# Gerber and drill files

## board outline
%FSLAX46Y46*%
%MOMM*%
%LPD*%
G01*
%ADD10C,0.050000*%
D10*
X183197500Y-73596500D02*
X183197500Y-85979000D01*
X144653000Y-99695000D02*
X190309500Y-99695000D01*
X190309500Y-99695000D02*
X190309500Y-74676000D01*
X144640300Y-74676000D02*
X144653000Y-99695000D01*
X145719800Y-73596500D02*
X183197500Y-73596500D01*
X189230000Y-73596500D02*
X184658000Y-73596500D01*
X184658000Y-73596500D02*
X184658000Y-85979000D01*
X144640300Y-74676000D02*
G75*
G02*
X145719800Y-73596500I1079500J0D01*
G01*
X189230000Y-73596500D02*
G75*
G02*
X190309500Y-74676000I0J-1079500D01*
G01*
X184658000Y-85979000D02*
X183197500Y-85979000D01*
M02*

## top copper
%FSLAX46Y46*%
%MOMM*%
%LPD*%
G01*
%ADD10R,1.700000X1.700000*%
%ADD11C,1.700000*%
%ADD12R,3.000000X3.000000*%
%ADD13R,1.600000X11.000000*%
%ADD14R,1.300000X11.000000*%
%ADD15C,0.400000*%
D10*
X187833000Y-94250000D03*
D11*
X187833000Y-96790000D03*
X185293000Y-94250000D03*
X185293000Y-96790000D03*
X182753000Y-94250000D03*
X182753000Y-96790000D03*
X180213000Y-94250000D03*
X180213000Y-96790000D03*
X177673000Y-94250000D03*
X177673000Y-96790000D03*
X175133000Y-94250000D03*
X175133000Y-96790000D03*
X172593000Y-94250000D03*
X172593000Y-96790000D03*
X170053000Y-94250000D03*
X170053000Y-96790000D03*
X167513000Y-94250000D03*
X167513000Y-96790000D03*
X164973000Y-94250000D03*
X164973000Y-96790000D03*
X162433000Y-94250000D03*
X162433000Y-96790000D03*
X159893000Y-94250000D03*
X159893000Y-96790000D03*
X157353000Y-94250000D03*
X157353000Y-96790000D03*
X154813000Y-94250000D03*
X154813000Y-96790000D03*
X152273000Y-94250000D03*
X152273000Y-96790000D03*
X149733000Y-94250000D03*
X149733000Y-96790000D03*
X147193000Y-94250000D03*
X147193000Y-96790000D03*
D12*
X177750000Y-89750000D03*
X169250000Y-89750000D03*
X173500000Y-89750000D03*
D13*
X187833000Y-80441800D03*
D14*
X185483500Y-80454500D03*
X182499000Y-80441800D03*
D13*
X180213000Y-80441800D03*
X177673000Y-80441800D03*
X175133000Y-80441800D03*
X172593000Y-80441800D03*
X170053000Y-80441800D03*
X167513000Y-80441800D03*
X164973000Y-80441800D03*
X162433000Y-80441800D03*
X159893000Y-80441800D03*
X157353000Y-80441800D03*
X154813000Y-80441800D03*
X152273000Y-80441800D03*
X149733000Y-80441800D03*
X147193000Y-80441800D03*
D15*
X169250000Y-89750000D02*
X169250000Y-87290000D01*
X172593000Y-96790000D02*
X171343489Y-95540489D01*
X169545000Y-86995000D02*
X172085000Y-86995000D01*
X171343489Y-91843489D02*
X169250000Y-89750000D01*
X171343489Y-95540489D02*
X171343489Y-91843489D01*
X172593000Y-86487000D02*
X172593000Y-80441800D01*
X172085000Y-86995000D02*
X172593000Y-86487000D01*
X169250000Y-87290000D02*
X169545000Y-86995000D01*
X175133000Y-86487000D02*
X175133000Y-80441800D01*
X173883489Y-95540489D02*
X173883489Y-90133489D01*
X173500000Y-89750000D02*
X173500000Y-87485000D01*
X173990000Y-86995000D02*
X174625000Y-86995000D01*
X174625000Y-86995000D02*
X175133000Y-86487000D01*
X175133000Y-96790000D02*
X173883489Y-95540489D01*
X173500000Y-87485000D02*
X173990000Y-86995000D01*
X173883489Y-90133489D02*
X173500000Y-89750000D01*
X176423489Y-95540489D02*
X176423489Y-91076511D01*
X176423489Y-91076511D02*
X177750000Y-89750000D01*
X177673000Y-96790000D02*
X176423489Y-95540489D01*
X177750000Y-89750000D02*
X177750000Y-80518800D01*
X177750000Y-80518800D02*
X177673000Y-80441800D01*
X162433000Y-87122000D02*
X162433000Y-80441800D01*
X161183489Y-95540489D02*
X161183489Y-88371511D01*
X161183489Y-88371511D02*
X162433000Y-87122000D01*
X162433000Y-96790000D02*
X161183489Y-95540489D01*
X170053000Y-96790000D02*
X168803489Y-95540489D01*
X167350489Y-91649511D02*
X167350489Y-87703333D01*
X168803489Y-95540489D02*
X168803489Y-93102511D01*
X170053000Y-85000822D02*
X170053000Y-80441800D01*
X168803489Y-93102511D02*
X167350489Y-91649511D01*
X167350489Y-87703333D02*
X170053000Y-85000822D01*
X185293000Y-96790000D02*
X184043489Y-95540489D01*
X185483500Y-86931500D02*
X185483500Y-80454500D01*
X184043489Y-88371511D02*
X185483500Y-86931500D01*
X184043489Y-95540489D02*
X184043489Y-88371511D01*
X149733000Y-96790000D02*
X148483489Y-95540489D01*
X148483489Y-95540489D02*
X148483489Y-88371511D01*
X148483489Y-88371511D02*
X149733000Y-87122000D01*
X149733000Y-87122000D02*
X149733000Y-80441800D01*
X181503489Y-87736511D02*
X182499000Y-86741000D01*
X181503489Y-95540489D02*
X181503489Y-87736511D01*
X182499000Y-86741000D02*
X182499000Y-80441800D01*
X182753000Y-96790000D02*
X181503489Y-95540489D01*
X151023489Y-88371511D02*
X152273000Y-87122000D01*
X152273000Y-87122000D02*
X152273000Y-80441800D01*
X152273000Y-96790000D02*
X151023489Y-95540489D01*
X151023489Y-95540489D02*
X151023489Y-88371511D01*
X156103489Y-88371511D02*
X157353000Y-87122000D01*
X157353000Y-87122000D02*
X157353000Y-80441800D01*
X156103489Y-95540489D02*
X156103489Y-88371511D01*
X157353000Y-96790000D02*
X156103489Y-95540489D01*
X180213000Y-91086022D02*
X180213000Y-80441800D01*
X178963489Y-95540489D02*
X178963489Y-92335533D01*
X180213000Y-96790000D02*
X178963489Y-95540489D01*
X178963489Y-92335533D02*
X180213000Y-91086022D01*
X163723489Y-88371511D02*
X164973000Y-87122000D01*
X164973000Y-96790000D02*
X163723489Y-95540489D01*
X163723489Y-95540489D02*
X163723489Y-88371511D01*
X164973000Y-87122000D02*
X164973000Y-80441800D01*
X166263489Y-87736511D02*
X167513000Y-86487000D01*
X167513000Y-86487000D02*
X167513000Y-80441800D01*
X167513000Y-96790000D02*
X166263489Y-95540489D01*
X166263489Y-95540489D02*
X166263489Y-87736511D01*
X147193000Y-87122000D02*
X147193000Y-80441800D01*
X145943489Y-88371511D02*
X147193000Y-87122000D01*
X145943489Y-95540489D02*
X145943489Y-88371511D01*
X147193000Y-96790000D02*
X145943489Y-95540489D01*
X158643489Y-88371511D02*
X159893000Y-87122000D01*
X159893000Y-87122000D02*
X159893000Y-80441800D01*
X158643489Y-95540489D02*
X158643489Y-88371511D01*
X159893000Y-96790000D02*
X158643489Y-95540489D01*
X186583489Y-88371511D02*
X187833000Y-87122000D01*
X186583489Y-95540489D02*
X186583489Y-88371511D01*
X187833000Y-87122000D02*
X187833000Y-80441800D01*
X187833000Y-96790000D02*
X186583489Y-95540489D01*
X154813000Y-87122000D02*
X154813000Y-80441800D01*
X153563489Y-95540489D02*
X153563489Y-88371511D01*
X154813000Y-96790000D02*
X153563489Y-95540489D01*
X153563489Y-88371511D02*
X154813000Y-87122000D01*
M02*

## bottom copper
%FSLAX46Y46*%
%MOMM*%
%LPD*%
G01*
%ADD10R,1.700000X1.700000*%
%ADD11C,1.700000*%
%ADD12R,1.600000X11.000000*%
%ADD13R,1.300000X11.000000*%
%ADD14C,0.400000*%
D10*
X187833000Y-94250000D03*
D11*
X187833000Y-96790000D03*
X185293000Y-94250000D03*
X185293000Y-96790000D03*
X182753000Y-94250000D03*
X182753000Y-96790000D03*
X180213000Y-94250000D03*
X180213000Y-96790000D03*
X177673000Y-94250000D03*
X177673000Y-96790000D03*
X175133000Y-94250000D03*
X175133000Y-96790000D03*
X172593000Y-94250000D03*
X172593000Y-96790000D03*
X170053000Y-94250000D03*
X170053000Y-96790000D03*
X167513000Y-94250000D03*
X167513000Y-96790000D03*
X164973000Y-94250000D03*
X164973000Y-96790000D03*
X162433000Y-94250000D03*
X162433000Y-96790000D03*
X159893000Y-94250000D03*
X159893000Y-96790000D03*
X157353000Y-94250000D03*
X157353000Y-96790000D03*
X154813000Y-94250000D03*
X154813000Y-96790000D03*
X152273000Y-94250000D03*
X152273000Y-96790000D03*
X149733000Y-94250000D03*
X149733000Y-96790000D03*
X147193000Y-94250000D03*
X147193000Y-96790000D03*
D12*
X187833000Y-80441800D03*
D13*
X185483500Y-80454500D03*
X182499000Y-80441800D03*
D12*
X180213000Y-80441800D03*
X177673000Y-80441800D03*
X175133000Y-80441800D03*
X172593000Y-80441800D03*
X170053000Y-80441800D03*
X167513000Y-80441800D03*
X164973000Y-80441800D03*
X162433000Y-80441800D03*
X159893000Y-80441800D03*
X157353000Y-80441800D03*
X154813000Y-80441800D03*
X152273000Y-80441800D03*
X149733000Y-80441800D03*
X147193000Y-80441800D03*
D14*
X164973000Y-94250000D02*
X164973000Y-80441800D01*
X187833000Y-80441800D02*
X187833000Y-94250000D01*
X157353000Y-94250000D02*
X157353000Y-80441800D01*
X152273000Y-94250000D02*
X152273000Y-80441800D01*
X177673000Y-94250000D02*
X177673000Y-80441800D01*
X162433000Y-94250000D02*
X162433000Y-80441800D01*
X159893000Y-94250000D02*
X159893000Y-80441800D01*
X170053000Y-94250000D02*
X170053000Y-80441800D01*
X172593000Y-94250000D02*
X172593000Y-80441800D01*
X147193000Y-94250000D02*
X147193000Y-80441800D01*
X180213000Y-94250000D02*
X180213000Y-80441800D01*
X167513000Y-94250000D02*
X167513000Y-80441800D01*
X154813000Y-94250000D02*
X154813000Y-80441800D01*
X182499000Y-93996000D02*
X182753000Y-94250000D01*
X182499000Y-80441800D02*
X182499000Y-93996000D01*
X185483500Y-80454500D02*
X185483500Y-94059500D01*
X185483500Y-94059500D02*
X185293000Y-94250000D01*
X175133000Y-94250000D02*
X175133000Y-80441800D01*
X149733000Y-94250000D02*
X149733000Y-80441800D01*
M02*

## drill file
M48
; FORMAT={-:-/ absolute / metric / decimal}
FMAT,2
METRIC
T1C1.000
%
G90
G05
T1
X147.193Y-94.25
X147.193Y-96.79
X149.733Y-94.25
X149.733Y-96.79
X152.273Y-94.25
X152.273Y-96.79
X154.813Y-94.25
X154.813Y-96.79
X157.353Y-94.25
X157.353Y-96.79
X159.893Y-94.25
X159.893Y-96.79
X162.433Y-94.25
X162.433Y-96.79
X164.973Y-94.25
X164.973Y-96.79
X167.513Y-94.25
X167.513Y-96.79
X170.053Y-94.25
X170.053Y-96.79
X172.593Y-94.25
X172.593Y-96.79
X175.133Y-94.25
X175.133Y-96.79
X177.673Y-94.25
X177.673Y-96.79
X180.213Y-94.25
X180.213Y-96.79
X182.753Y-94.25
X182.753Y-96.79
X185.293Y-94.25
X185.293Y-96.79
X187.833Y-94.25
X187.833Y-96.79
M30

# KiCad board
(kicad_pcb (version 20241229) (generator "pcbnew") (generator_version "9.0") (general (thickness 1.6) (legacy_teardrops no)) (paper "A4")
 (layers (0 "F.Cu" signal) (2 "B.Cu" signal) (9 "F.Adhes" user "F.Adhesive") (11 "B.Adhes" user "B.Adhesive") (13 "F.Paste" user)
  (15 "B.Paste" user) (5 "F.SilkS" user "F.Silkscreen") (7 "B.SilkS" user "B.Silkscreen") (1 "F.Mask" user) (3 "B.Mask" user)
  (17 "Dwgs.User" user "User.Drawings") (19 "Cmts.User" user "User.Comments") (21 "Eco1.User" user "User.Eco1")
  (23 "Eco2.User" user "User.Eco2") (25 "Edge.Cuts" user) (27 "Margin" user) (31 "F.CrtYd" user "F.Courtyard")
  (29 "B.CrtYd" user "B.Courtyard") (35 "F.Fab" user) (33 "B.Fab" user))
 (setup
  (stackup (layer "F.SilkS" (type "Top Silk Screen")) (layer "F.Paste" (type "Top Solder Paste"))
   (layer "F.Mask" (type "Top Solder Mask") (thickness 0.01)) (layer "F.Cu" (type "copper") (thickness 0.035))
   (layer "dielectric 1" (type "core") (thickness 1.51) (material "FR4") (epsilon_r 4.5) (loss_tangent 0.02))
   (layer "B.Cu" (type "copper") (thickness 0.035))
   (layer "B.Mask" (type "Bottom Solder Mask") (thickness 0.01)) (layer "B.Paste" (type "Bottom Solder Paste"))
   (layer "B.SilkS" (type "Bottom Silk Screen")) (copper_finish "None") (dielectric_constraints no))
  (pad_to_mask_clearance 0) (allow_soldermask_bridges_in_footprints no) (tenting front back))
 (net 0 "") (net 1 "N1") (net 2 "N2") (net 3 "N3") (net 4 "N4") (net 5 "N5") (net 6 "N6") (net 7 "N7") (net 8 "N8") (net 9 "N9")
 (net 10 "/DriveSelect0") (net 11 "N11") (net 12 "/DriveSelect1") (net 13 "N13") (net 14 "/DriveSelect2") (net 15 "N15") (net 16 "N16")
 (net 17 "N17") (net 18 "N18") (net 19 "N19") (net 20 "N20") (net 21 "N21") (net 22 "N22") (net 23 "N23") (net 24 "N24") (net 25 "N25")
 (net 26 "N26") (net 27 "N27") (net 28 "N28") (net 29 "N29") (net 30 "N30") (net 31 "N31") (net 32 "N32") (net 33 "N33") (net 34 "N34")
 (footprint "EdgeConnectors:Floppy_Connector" (layer "F.Cu") (at 187.833 94.25 -90)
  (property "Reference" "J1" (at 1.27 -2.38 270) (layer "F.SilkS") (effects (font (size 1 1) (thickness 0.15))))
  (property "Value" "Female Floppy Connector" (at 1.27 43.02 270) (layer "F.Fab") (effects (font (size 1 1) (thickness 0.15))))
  (pad "1" thru_hole rect (at 0 0 270) (size 1.7 1.7) (drill 1) (layers "*.Cu" "*.Mask") (remove_unused_layers no) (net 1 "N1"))
  (pad "2" thru_hole circle (at 2.54 0 270) (size 1.7 1.7) (drill 1) (layers "*.Cu" "*.Mask") (remove_unused_layers no) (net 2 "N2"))
  (pad "3" thru_hole circle (at 0 2.54 270) (size 1.7 1.7) (drill 1) (layers "*.Cu" "*.Mask") (remove_unused_layers no) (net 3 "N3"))
  (pad "4" thru_hole circle (at 2.54 2.54 270) (size 1.7 1.7) (drill 1) (layers "*.Cu" "*.Mask") (remove_unused_layers no) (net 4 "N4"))
  (pad "5" thru_hole circle (at 0 5.08 270) (size 1.7 1.7) (drill 1) (layers "*.Cu" "*.Mask") (remove_unused_layers no) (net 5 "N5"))
  (pad "6" thru_hole circle (at 2.54 5.08 270) (size 1.7 1.7) (drill 1) (layers "*.Cu" "*.Mask") (remove_unused_layers no) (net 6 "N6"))
  (pad "7" thru_hole circle (at 0 7.62 270) (size 1.7 1.7) (drill 1) (layers "*.Cu" "*.Mask") (remove_unused_layers no) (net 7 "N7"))
  (pad "8" thru_hole circle (at 2.54 7.62 270) (size 1.7 1.7) (drill 1) (layers "*.Cu" "*.Mask") (remove_unused_layers no) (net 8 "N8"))
  (pad "9" thru_hole circle (at 0 10.16 270) (size 1.7 1.7) (drill 1) (layers "*.Cu" "*.Mask") (remove_unused_layers no) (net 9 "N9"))
  (pad "10" thru_hole circle (at 2.54 10.16 270) (size 1.7 1.7) (drill 1) (layers "*.Cu" "*.Mask") (remove_unused_layers no)
   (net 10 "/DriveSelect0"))
  (pad "11" thru_hole circle (at 0 12.7 270) (size 1.7 1.7) (drill 1) (layers "*.Cu" "*.Mask") (remove_unused_layers no) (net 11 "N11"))
  (pad "12" thru_hole circle (at 2.54 12.7 270) (size 1.7 1.7) (drill 1) (layers "*.Cu" "*.Mask") (remove_unused_layers no)
   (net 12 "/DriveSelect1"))
  (pad "13" thru_hole circle (at 0 15.24 270) (size 1.7 1.7) (drill 1) (layers "*.Cu" "*.Mask") (remove_unused_layers no) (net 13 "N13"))
  (pad "14" thru_hole circle (at 2.54 15.24 270) (size 1.7 1.7) (drill 1) (layers "*.Cu" "*.Mask") (remove_unused_layers no)
   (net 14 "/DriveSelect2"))
  (pad "15" thru_hole circle (at 0 17.78 270) (size 1.7 1.7) (drill 1) (layers "*.Cu" "*.Mask") (remove_unused_layers no) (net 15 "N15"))
  (pad "16" thru_hole circle (at 2.54 17.78 270) (size 1.7 1.7) (drill 1) (layers "*.Cu" "*.Mask") (remove_unused_layers no) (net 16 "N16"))
  (pad "17" thru_hole circle (at 0 20.32 270) (size 1.7 1.7) (drill 1) (layers "*.Cu" "*.Mask") (remove_unused_layers no) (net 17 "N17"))
  (pad "18" thru_hole circle (at 2.54 20.32 270) (size 1.7 1.7) (drill 1) (layers "*.Cu" "*.Mask") (remove_unused_layers no) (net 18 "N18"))
  (pad "19" thru_hole circle (at 0 22.86 270) (size 1.7 1.7) (drill 1) (layers "*.Cu" "*.Mask") (remove_unused_layers no) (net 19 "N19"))
  (pad "20" thru_hole circle (at 2.54 22.86 270) (size 1.7 1.7) (drill 1) (layers "*.Cu" "*.Mask") (remove_unused_layers no) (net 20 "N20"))
  (pad "21" thru_hole circle (at 0 25.4 270) (size 1.7 1.7) (drill 1) (layers "*.Cu" "*.Mask") (remove_unused_layers no) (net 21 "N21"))
  (pad "22" thru_hole circle (at 2.54 25.4 270) (size 1.7 1.7) (drill 1) (layers "*.Cu" "*.Mask") (remove_unused_layers no) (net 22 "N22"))
  (pad "23" thru_hole circle (at 0 27.94 270) (size 1.7 1.7) (drill 1) (layers "*.Cu" "*.Mask") (remove_unused_layers no) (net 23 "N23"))
  (pad "24" thru_hole circle (at 2.54 27.94 270) (size 1.7 1.7) (drill 1) (layers "*.Cu" "*.Mask") (remove_unused_layers no) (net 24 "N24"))
  (pad "25" thru_hole circle (at 0 30.48 270) (size 1.7 1.7) (drill 1) (layers "*.Cu" "*.Mask") (remove_unused_layers no) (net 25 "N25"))
  (pad "26" thru_hole circle (at 2.54 30.48 270) (size 1.7 1.7) (drill 1) (layers "*.Cu" "*.Mask") (remove_unused_layers no) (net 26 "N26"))
  (pad "27" thru_hole circle (at 0 33.02 270) (size 1.7 1.7) (drill 1) (layers "*.Cu" "*.Mask") (remove_unused_layers no) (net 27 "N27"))
  (pad "28" thru_hole circle (at 2.54 33.02 270) (size 1.7 1.7) (drill 1) (layers "*.Cu" "*.Mask") (remove_unused_layers no) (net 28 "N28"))
  (pad "29" thru_hole circle (at 0 35.56 270) (size 1.7 1.7) (drill 1) (layers "*.Cu" "*.Mask") (remove_unused_layers no) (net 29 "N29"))
  (pad "30" thru_hole circle (at 2.54 35.56 270) (size 1.7 1.7) (drill 1) (layers "*.Cu" "*.Mask") (remove_unused_layers no) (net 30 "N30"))
  (pad "31" thru_hole circle (at 0 38.1 270) (size 1.7 1.7) (drill 1) (layers "*.Cu" "*.Mask") (remove_unused_layers no) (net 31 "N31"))
  (pad "32" thru_hole circle (at 2.54 38.1 270) (size 1.7 1.7) (drill 1) (layers "*.Cu" "*.Mask") (remove_unused_layers no) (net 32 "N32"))
  (pad "33" thru_hole circle (at 0 40.64 270) (size 1.7 1.7) (drill 1) (layers "*.Cu" "*.Mask") (remove_unused_layers no) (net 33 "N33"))
  (pad "34" thru_hole circle (at 2.54 40.64 270) (size 1.7 1.7) (drill 1) (layers "*.Cu" "*.Mask") (remove_unused_layers no) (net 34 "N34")))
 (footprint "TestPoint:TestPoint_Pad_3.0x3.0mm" (layer "F.Cu") (at 177.75 89.75)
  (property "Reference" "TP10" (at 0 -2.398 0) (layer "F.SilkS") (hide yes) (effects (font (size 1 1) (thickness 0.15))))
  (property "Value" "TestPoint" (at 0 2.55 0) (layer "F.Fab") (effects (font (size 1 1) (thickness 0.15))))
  (pad "1" smd rect (at 0 0) (size 3 3) (layers "F.Cu" "F.Mask") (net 10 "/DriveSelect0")))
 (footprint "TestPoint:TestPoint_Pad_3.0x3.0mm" (layer "F.Cu") (at 169.25 89.75)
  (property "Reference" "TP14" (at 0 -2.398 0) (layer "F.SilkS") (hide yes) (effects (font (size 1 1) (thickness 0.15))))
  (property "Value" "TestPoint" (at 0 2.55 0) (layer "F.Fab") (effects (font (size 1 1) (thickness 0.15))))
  (pad "1" smd rect (at 0 0) (size 3 3) (layers "F.Cu" "F.Mask") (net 14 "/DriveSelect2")))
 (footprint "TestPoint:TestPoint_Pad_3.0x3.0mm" (layer "F.Cu") (at 173.5 89.75)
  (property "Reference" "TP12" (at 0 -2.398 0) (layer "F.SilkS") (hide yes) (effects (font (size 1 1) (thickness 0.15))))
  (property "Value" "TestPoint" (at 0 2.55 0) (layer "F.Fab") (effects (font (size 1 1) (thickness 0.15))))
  (pad "1" smd rect (at 0 0) (size 3 3) (layers "F.Cu" "F.Mask") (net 12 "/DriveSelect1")))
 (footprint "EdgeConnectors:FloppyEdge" (layer "B.Cu") (at 167.513 71.501)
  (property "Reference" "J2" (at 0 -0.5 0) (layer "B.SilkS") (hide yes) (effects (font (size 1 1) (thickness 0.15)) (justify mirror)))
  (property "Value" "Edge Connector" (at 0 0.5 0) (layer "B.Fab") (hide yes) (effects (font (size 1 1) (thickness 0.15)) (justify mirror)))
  (pad "1" smd rect (at 20.32 8.9408) (size 1.6 11) (layers "B.Cu" "B.Mask" "B.Paste") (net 1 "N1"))
  (pad "2" smd rect (at 20.32 8.9408) (size 1.6 11) (layers "F.Cu" "F.Mask" "F.Paste") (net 2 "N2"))
  (pad "3" smd rect (at 17.9705 8.9535) (size 1.3 11) (layers "B.Cu" "B.Mask" "B.Paste") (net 3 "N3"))
  (pad "4" smd rect (at 17.9705 8.9535) (size 1.3 11) (layers "F.Cu" "F.Mask" "F.Paste") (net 4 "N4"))
  (pad "5" smd rect (at 14.986 8.9408) (size 1.3 11) (layers "B.Cu" "B.Mask" "B.Paste") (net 5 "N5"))
  (pad "6" smd rect (at 14.986 8.9408) (size 1.3 11) (layers "F.Cu" "F.Mask" "F.Paste") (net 6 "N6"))
  (pad "7" smd rect (at 12.7 8.9408) (size 1.6 11) (layers "B.Cu" "B.Mask" "B.Paste") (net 7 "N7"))
  (pad "8" smd rect (at 12.7 8.9408) (size 1.6 11) (layers "F.Cu" "F.Mask" "F.Paste") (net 8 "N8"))
  (pad "9" smd rect (at 10.16 8.9408) (size 1.6 11) (layers "B.Cu" "B.Mask" "B.Paste") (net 9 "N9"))
  (pad "10" smd rect (at 10.16 8.9408) (size 1.6 11) (layers "F.Cu" "F.Mask" "F.Paste") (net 10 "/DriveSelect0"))
  (pad "11" smd rect (at 7.62 8.9408) (size 1.6 11) (layers "B.Cu" "B.Mask" "B.Paste") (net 11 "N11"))
  (pad "12" smd rect (at 7.62 8.9408) (size 1.6 11) (layers "F.Cu" "F.Mask" "F.Paste") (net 12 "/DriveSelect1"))
  (pad "13" smd rect (at 5.08 8.9408) (size 1.6 11) (layers "B.Cu" "B.Mask" "B.Paste") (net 13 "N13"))
  (pad "14" smd rect (at 5.08 8.9408) (size 1.6 11) (layers "F.Cu" "F.Mask" "F.Paste") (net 14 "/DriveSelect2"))
  (pad "15" smd rect (at 2.54 8.9408) (size 1.6 11) (layers "B.Cu" "B.Mask" "B.Paste") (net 15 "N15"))
  (pad "16" smd rect (at 2.54 8.9408) (size 1.6 11) (layers "F.Cu" "F.Mask" "F.Paste") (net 16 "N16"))
  (pad "17" smd rect (at 0 8.9408) (size 1.6 11) (layers "B.Cu" "B.Mask" "B.Paste") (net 17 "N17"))
  (pad "18" smd rect (at 0 8.9408) (size 1.6 11) (layers "F.Cu" "F.Mask" "F.Paste") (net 18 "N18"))
  (pad "19" smd rect (at -2.54 8.9408) (size 1.6 11) (layers "B.Cu" "B.Mask" "B.Paste") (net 19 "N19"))
  (pad "20" smd rect (at -2.54 8.9408) (size 1.6 11) (layers "F.Cu" "F.Mask" "F.Paste") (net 20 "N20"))
  (pad "21" smd rect (at -5.08 8.9408) (size 1.6 11) (layers "B.Cu" "B.Mask" "B.Paste") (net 21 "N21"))
  (pad "22" smd rect (at -5.08 8.9408) (size 1.6 11) (layers "F.Cu" "F.Mask" "F.Paste") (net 22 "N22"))
  (pad "23" smd rect (at -7.62 8.9408) (size 1.6 11) (layers "B.Cu" "B.Mask" "B.Paste") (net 23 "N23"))
  (pad "24" smd rect (at -7.62 8.9408) (size 1.6 11) (layers "F.Cu" "F.Mask" "F.Paste") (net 24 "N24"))
  (pad "25" smd rect (at -10.16 8.9408) (size 1.6 11) (layers "B.Cu" "B.Mask" "B.Paste") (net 25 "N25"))
  (pad "26" smd rect (at -10.16 8.9408) (size 1.6 11) (layers "F.Cu" "F.Mask" "F.Paste") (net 26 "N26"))
  (pad "27" smd rect (at -12.7 8.9408) (size 1.6 11) (layers "B.Cu" "B.Mask" "B.Paste") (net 27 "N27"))
  (pad "28" smd rect (at -12.7 8.9408) (size 1.6 11) (layers "F.Cu" "F.Mask" "F.Paste") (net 28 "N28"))
  (pad "29" smd rect (at -15.24 8.9408) (size 1.6 11) (layers "B.Cu" "B.Mask" "B.Paste") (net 29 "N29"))
  (pad "30" smd rect (at -15.24 8.9408) (size 1.6 11) (layers "F.Cu" "F.Mask" "F.Paste") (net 30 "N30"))
  (pad "31" smd rect (at -17.78 8.9408) (size 1.6 11) (layers "B.Cu" "B.Mask" "B.Paste") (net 31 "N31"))
  (pad "32" smd rect (at -17.78 8.9408) (size 1.6 11) (layers "F.Cu" "F.Mask" "F.Paste") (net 32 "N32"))
  (pad "33" smd rect (at -20.32 8.9408) (size 1.6 11) (layers "B.Cu" "B.Mask" "B.Paste") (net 33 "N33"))
  (pad "34" smd rect (at -20.32 8.9408) (size 1.6 11) (layers "F.Cu" "F.Mask" "F.Paste") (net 34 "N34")))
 (gr_line (start 183.1975 73.5965) (end 183.1975 85.979) (stroke (width 0.05) (type solid)) (layer "Edge.Cuts"))
 (gr_line (start 144.653 99.695) (end 190.3095 99.695) (stroke (width 0.05) (type solid)) (layer "Edge.Cuts"))
 (gr_line (start 190.3095 99.695) (end 190.3095 74.676) (stroke (width 0.05) (type default)) (layer "Edge.Cuts"))
 (gr_line (start 144.6403 74.676) (end 144.653 99.695) (stroke (width 0.05) (type default)) (layer "Edge.Cuts"))
 (gr_line (start 145.7198 73.5965) (end 183.1975 73.5965) (stroke (width 0.05) (type default)) (layer "Edge.Cuts"))
 (gr_line (start 189.23 73.5965) (end 184.658 73.5965) (stroke (width 0.05) (type default)) (layer "Edge.Cuts"))
 (gr_line (start 184.658 73.5965) (end 184.658 85.979) (stroke (width 0.05) (type solid)) (layer "Edge.Cuts"))
 (gr_arc (start 144.6403 74.676) (mid 144.956478 73.912678) (end 145.7198 73.5965) (stroke (width 0.05) (type default)) (layer "Edge.Cuts"))
 (gr_arc (start 189.23 73.5965) (mid 189.993322 73.912678) (end 190.3095 74.676) (stroke (width 0.05) (type default)) (layer "Edge.Cuts"))
 (gr_line (start 184.658 85.979) (end 183.1975 85.979) (stroke (width 0.05) (type solid)) (layer "Edge.Cuts"))
 (segment (start 169.25 89.75) (end 169.25 87.29) (width 0.4) (layer "F.Cu") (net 14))
 (segment (start 172.593 96.79) (end 171.343489 95.540489) (width 0.4) (layer "F.Cu") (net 14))
 (segment (start 169.545 86.995) (end 172.085 86.995) (width 0.4) (layer "F.Cu") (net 14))
 (segment (start 171.343489 91.843489) (end 169.25 89.75) (width 0.4) (layer "F.Cu") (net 14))
 (segment (start 171.343489 95.540489) (end 171.343489 91.843489) (width 0.4) (layer "F.Cu") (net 14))
 (segment (start 172.593 86.487) (end 172.593 80.4418) (width 0.4) (layer "F.Cu") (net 14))
 (segment (start 172.085 86.995) (end 172.593 86.487) (width 0.4) (layer "F.Cu") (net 14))
 (segment (start 169.25 87.29) (end 169.545 86.995) (width 0.4) (layer "F.Cu") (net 14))
 (segment (start 175.133 86.487) (end 175.133 80.4418) (width 0.4) (layer "F.Cu") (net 12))
 (segment (start 173.883489 95.540489) (end 173.883489 90.133489) (width 0.4) (layer "F.Cu") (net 12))
 (segment (start 173.5 89.75) (end 173.5 87.485) (width 0.4) (layer "F.Cu") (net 12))
 (segment (start 173.99 86.995) (end 174.625 86.995) (width 0.4) (layer "F.Cu") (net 12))
 (segment (start 174.625 86.995) (end 175.133 86.487) (width 0.4) (layer "F.Cu") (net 12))
 (segment (start 175.133 96.79) (end 173.883489 95.540489) (width 0.4) (layer "F.Cu") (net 12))
 (segment (start 173.5 87.485) (end 173.99 86.995) (width 0.4) (layer "F.Cu") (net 12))
 (segment (start 173.883489 90.133489) (end 173.5 89.75) (width 0.4) (layer "F.Cu") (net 12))
 (segment (start 176.423489 95.540489) (end 176.423489 91.076511) (width 0.4) (layer "F.Cu") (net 10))
 (segment (start 176.423489 91.076511) (end 177.75 89.75) (width 0.4) (layer "F.Cu") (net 10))
 (segment (start 177.673 96.79) (end 176.423489 95.540489) (width 0.4) (layer "F.Cu") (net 10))
 (segment (start 177.75 89.75) (end 177.75 80.5188) (width 0.4) (layer "F.Cu") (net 10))
 (segment (start 177.75 80.5188) (end 177.673 80.4418) (width 0.4) (layer "F.Cu") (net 10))
 (segment (start 164.973 94.25) (end 164.973 80.4418) (width 0.4) (layer "B.Cu") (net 19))
 (segment (start 162.433 87.122) (end 162.433 80.4418) (width 0.4) (layer "F.Cu") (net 22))
 (segment (start 161.183489 95.540489) (end 161.183489 88.371511) (width 0.4) (layer "F.Cu") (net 22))
 (segment (start 161.183489 88.371511) (end 162.433 87.122) (width 0.4) (layer "F.Cu") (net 22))
 (segment (start 162.433 96.79) (end 161.183489 95.540489) (width 0.4) (layer "F.Cu") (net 22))
 (segment (start 170.053 96.79) (end 168.803489 95.540489) (width 0.4) (layer "F.Cu") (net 16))
 (segment (start 167.350489 91.649511) (end 167.350489 87.703333) (width 0.4) (layer "F.Cu") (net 16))
 (segment (start 168.803489 95.540489) (end 168.803489 93.102511) (width 0.4) (layer "F.Cu") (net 16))
 (segment (start 170.053 85.000822) (end 170.053 80.4418) (width 0.4) (layer "F.Cu") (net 16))
 (segment (start 168.803489 93.102511) (end 167.350489 91.649511) (width 0.4) (layer "F.Cu") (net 16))
 (segment (start 167.350489 87.703333) (end 170.053 85.000822) (width 0.4) (layer "F.Cu") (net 16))
 (segment (start 187.833 80.4418) (end 187.833 94.25) (width 0.4) (layer "B.Cu") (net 1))
 (segment (start 185.293 96.79) (end 184.043489 95.540489) (width 0.4) (layer "F.Cu") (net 4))
 (segment (start 185.4835 86.9315) (end 185.4835 80.4545) (width 0.4) (layer "F.Cu") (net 4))
 (segment (start 184.043489 88.371511) (end 185.4835 86.9315) (width 0.4) (layer "F.Cu") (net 4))
 (segment (start 184.043489 95.540489) (end 184.043489 88.371511) (width 0.4) (layer "F.Cu") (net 4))
 (segment (start 157.353 94.25) (end 157.353 80.4418) (width 0.4) (layer "B.Cu") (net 25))
 (segment (start 152.273 94.25) (end 152.273 80.4418) (width 0.4) (layer "B.Cu") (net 29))
 (segment (start 149.733 96.79) (end 148.483489 95.540489) (width 0.4) (layer "F.Cu") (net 32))
 (segment (start 148.483489 95.540489) (end 148.483489 88.371511) (width 0.4) (layer "F.Cu") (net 32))
 (segment (start 148.483489 88.371511) (end 149.733 87.122) (width 0.4) (layer "F.Cu") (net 32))
 (segment (start 149.733 87.122) (end 149.733 80.4418) (width 0.4) (layer "F.Cu") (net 32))
 (segment (start 181.503489 87.736511) (end 182.499 86.741) (width 0.4) (layer "F.Cu") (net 6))
 (segment (start 181.503489 95.540489) (end 181.503489 87.736511) (width 0.4) (layer "F.Cu") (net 6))
 (segment (start 182.499 86.741) (end 182.499 80.4418) (width 0.4) (layer "F.Cu") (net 6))
 (segment (start 182.753 96.79) (end 181.503489 95.540489) (width 0.4) (layer "F.Cu") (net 6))
 (segment (start 151.023489 88.371511) (end 152.273 87.122) (width 0.4) (layer "F.Cu") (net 30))
 (segment (start 152.273 87.122) (end 152.273 80.4418) (width 0.4) (layer "F.Cu") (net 30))
 (segment (start 152.273 96.79) (end 151.023489 95.540489) (width 0.4) (layer "F.Cu") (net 30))
 (segment (start 151.023489 95.540489) (end 151.023489 88.371511) (width 0.4) (layer "F.Cu") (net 30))
 (segment (start 177.673 94.25) (end 177.673 80.4418) (width 0.4) (layer "B.Cu") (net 9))
 (segment (start 156.103489 88.371511) (end 157.353 87.122) (width 0.4) (layer "F.Cu") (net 26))
 (segment (start 157.353 87.122) (end 157.353 80.4418) (width 0.4) (layer "F.Cu") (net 26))
 (segment (start 156.103489 95.540489) (end 156.103489 88.371511) (width 0.4) (layer "F.Cu") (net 26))
 (segment (start 157.353 96.79) (end 156.103489 95.540489) (width 0.4) (layer "F.Cu") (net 26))
 (segment (start 162.433 94.25) (end 162.433 80.4418) (width 0.4) (layer "B.Cu") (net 21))
 (segment (start 159.893 94.25) (end 159.893 80.4418) (width 0.4) (layer "B.Cu") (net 23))
 (segment (start 180.213 91.086022) (end 180.213 80.4418) (width 0.4) (layer "F.Cu") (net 8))
 (segment (start 178.963489 95.540489) (end 178.963489 92.335533) (width 0.4) (layer "F.Cu") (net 8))
 (segment (start 180.213 96.79) (end 178.963489 95.540489) (width 0.4) (layer "F.Cu") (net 8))
 (segment (start 178.963489 92.335533) (end 180.213 91.086022) (width 0.4) (layer "F.Cu") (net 8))
 (segment (start 163.723489 88.371511) (end 164.973 87.122) (width 0.4) (layer "F.Cu") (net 20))
 (segment (start 164.973 96.79) (end 163.723489 95.540489) (width 0.4) (layer "F.Cu") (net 20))
 (segment (start 163.723489 95.540489) (end 163.723489 88.371511) (width 0.4) (layer "F.Cu") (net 20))
 (segment (start 164.973 87.122) (end 164.973 80.4418) (width 0.4) (layer "F.Cu") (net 20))
 (segment (start 170.053 94.25) (end 170.053 80.4418) (width 0.4) (layer "B.Cu") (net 15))
 (segment (start 172.593 94.25) (end 172.593 80.4418) (width 0.4) (layer "B.Cu") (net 13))
 (segment (start 147.193 94.25) (end 147.193 80.4418) (width 0.4) (layer "B.Cu") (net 33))
 (segment (start 180.213 94.25) (end 180.213 80.4418) (width 0.4) (layer "B.Cu") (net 7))
 (segment (start 167.513 94.25) (end 167.513 80.4418) (width 0.4) (layer "B.Cu") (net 17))
 (segment (start 154.813 94.25) (end 154.813 80.4418) (width 0.4) (layer "B.Cu") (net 27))
 (segment (start 182.499 93.996) (end 182.753 94.25) (width 0.4) (layer "B.Cu") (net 5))
 (segment (start 182.499 80.4418) (end 182.499 93.996) (width 0.4) (layer "B.Cu") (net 5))
 (segment (start 185.4835 80.4545) (end 185.4835 94.0595) (width 0.4) (layer "B.Cu") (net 3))
 (segment (start 185.4835 94.0595) (end 185.293 94.25) (width 0.4) (layer "B.Cu") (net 3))
 (segment (start 166.263489 87.736511) (end 167.513 86.487) (width 0.4) (layer "F.Cu") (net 18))
 (segment (start 167.513 86.487) (end 167.513 80.4418) (width 0.4) (layer "F.Cu") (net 18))
 (segment (start 167.513 96.79) (end 166.263489 95.540489) (width 0.4) (layer "F.Cu") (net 18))
 (segment (start 166.263489 95.540489) (end 166.263489 87.736511) (width 0.4) (layer "F.Cu") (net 18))
 (segment (start 147.193 87.122) (end 147.193 80.4418) (width 0.4) (layer "F.Cu") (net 34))
 (segment (start 145.943489 88.371511) (end 147.193 87.122) (width 0.4) (layer "F.Cu") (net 34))
 (segment (start 145.943489 95.540489) (end 145.943489 88.371511) (width 0.4) (layer "F.Cu") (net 34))
 (segment (start 147.193 96.79) (end 145.943489 95.540489) (width 0.4) (layer "F.Cu") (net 34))
 (segment (start 158.643489 88.371511) (end 159.893 87.122) (width 0.4) (layer "F.Cu") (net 24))
 (segment (start 159.893 87.122) (end 159.893 80.4418) (width 0.4) (layer "F.Cu") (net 24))
 (segment (start 158.643489 95.540489) (end 158.643489 88.371511) (width 0.4) (layer "F.Cu") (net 24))
 (segment (start 159.893 96.79) (end 158.643489 95.540489) (width 0.4) (layer "F.Cu") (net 24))
 (segment (start 175.133 94.25) (end 175.133 80.4418) (width 0.4) (layer "B.Cu") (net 11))
 (segment (start 149.733 94.25) (end 149.733 80.4418) (width 0.4) (layer "B.Cu") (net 31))
 (segment (start 186.583489 88.371511) (end 187.833 87.122) (width 0.4) (layer "F.Cu") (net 2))
 (segment (start 186.583489 95.540489) (end 186.583489 88.371511) (width 0.4) (layer "F.Cu") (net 2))
 (segment (start 187.833 87.122) (end 187.833 80.4418) (width 0.4) (layer "F.Cu") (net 2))
 (segment (start 187.833 96.79) (end 186.583489 95.540489) (width 0.4) (layer "F.Cu") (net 2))
 (segment (start 154.813 87.122) (end 154.813 80.4418) (width 0.4) (layer "F.Cu") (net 28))
 (segment (start 153.563489 95.540489) (end 153.563489 88.371511) (width 0.4) (layer "F.Cu") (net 28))
 (segment (start 154.813 96.79) (end 153.563489 95.540489) (width 0.4) (layer "F.Cu") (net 28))
 (segment (start 153.563489 88.371511) (end 154.813 87.122) (width 0.4) (layer "F.Cu") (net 28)))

